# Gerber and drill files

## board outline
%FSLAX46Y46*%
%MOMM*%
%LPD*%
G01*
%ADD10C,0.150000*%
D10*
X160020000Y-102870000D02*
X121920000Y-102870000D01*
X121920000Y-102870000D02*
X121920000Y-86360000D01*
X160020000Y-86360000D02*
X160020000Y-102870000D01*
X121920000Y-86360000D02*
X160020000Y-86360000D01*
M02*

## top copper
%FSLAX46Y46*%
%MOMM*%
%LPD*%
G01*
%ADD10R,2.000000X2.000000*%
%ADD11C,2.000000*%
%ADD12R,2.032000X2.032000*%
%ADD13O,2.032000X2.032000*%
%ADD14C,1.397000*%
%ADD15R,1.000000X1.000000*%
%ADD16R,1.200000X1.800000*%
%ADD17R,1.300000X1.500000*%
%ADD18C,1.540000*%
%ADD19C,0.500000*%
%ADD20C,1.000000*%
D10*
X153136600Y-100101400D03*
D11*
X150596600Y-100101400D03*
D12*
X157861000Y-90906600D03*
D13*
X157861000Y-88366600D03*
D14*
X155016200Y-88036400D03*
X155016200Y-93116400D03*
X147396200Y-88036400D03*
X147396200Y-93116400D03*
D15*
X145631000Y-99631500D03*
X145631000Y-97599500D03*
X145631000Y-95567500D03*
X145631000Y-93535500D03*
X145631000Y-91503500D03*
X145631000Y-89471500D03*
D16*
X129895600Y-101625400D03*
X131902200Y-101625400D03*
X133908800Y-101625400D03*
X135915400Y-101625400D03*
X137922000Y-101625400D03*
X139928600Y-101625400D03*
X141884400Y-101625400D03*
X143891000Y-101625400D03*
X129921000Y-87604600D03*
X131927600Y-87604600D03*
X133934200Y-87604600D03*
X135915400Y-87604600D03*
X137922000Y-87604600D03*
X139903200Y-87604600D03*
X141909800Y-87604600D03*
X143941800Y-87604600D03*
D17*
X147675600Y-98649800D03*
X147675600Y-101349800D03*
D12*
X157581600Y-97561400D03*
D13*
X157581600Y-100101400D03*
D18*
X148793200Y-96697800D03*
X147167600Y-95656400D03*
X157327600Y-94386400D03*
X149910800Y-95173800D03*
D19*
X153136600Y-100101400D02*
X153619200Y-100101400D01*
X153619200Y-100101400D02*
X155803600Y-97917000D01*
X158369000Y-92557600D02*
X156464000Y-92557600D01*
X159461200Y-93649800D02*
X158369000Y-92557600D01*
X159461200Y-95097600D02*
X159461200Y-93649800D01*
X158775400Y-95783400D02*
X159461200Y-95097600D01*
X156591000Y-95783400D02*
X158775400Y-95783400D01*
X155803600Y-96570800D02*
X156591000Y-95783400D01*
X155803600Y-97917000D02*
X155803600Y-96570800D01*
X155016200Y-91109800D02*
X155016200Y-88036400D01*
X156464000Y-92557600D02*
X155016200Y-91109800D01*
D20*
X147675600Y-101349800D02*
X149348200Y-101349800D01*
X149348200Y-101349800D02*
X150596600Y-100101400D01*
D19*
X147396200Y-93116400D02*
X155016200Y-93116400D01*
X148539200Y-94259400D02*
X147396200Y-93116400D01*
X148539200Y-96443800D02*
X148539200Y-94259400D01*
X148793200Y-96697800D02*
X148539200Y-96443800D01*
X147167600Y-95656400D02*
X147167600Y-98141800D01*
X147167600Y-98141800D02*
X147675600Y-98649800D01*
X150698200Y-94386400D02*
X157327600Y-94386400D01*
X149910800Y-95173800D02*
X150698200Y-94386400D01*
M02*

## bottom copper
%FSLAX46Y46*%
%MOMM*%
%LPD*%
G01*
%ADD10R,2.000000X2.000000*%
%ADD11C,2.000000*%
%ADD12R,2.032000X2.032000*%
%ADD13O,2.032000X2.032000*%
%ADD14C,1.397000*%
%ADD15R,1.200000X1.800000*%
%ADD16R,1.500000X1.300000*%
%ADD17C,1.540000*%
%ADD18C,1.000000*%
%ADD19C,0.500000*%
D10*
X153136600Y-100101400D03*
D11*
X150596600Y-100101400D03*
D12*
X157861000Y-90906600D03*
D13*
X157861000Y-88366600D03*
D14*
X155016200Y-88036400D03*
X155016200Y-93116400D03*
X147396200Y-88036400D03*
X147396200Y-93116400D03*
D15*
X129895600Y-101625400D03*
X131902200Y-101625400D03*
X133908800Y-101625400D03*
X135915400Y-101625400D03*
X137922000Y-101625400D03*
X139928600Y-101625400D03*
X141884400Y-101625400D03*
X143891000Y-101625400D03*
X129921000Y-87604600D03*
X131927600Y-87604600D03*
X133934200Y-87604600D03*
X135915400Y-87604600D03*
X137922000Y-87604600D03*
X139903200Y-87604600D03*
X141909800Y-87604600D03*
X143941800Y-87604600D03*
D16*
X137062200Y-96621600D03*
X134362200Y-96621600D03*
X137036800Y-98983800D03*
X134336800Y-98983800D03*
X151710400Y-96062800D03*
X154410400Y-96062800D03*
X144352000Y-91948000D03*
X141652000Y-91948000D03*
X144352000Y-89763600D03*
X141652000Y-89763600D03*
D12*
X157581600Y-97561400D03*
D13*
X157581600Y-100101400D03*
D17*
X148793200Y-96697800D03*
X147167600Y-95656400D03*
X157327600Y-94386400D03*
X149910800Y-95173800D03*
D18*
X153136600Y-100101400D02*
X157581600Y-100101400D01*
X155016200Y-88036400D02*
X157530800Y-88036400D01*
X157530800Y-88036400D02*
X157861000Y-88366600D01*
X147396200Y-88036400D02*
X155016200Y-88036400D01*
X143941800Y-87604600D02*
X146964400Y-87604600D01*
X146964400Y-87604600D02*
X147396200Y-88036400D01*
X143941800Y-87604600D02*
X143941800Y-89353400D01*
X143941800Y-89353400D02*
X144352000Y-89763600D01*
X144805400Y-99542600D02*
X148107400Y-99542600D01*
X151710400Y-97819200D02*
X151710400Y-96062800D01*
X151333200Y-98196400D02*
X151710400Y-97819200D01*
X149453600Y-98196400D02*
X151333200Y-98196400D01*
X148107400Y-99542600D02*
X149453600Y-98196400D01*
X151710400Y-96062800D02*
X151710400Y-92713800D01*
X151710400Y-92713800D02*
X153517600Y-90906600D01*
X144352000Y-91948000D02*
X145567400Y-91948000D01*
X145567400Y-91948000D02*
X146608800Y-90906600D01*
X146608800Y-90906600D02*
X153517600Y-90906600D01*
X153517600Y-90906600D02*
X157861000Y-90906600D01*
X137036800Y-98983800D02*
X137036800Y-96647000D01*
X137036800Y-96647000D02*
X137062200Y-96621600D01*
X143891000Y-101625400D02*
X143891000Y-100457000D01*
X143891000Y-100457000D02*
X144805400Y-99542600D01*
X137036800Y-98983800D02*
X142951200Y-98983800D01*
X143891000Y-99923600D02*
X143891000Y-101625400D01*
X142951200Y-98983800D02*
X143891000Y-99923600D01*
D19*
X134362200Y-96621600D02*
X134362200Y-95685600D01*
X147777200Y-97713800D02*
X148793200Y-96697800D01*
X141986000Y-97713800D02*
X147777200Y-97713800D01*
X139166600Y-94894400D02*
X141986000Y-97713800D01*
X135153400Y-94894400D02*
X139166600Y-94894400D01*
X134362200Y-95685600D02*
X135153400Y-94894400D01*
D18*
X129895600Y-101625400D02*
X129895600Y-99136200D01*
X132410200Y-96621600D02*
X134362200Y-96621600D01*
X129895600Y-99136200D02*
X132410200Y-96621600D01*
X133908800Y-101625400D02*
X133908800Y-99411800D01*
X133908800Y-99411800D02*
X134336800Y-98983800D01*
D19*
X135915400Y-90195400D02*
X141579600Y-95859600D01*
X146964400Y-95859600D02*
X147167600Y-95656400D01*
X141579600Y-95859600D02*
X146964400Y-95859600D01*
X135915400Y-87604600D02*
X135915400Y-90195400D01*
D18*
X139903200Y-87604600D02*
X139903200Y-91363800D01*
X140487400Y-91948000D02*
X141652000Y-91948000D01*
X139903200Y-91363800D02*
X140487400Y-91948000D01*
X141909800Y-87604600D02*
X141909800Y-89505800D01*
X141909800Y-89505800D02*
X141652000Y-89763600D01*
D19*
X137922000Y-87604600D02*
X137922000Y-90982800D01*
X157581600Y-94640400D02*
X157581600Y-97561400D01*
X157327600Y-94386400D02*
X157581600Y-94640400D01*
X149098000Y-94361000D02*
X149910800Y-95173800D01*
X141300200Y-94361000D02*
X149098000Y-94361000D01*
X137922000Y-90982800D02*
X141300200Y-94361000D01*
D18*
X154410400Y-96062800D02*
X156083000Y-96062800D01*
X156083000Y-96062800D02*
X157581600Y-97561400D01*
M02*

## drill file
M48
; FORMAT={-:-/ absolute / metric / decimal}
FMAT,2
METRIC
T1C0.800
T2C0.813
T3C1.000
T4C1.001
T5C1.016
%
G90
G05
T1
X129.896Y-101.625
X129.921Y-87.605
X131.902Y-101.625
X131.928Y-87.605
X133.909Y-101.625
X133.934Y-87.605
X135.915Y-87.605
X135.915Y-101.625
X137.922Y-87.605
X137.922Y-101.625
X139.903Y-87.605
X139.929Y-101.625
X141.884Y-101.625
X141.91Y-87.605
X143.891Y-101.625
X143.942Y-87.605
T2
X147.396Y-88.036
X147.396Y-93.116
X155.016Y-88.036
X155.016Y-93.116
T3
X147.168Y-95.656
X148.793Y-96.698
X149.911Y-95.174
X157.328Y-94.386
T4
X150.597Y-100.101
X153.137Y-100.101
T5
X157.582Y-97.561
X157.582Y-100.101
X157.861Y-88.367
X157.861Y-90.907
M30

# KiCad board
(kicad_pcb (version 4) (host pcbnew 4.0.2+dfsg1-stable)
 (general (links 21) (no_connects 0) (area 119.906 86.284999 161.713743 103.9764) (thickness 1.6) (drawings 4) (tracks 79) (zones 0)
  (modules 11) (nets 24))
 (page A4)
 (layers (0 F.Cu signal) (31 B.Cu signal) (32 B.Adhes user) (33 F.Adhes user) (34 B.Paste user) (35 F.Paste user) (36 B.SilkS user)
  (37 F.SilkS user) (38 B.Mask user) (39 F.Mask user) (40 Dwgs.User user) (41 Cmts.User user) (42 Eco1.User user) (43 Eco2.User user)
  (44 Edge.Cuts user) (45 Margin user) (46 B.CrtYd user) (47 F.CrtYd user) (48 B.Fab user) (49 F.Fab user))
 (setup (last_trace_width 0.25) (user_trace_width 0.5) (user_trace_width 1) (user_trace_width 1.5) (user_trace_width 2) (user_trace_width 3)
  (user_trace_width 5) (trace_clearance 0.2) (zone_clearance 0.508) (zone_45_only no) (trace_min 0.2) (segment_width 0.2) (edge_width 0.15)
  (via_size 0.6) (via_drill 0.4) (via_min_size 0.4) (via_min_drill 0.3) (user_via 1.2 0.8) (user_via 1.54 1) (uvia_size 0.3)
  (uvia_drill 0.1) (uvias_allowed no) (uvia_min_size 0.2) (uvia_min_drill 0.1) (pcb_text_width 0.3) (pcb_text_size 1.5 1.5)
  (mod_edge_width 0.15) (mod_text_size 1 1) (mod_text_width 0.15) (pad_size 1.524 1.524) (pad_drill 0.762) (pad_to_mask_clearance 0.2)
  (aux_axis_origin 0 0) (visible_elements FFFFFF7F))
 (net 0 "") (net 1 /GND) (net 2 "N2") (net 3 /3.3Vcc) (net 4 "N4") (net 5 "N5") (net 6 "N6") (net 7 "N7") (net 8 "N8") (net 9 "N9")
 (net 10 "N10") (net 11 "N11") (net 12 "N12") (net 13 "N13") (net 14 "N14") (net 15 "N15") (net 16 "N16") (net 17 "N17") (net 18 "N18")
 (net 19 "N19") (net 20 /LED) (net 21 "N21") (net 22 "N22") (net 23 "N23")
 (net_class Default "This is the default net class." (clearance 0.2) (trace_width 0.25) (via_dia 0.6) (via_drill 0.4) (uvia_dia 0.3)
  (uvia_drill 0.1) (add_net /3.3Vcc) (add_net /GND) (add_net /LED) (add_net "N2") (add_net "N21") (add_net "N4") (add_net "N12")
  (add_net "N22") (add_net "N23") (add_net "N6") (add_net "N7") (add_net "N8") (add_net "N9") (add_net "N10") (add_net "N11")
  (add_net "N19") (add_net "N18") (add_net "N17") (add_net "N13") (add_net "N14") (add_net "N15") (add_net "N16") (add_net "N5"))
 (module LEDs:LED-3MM (layer F.Cu) (at 153.1366 100.1014 180)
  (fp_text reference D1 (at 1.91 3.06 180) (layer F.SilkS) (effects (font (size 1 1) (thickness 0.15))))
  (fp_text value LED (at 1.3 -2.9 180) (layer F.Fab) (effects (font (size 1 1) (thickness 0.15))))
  (pad 1 thru_hole rect (at 0 0 270) (size 2 2) (drill 1.00076) (layers *.Cu *.Mask F.SilkS) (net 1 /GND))
  (pad 2 thru_hole circle (at 2.54 0 180) (size 2 2) (drill 1.00076) (layers *.Cu *.Mask F.SilkS) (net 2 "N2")))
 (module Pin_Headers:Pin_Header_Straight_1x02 (layer F.Cu) (at 157.861 90.9066 180)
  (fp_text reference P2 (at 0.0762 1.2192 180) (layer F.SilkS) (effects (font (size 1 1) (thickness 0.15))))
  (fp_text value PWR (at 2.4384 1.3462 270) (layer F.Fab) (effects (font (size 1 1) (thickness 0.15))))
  (pad 1 thru_hole rect (at 0 0 180) (size 2.032 2.032) (drill 1.016) (layers *.Cu *.Mask F.SilkS) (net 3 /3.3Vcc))
  (pad 2 thru_hole oval (at 0 2.54 180) (size 2.032 2.032) (drill 1.016) (layers *.Cu *.Mask F.SilkS) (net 1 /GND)))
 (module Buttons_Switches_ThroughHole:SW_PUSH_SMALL (layer F.Cu) (at 151.2062 90.5764)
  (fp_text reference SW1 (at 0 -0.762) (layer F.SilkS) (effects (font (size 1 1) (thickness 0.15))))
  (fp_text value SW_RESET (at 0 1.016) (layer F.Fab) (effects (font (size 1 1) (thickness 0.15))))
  (pad 1 thru_hole circle (at 3.81 -2.54) (size 1.397 1.397) (drill 0.8128) (layers *.Cu *.Mask F.SilkS) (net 1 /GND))
  (pad 2 thru_hole circle (at 3.81 2.54) (size 1.397 1.397) (drill 0.8128) (layers *.Cu *.Mask F.SilkS) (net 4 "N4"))
  (pad 1 thru_hole circle (at -3.81 -2.54) (size 1.397 1.397) (drill 0.8128) (layers *.Cu *.Mask F.SilkS) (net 1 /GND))
  (pad 2 thru_hole circle (at -3.81 2.54) (size 1.397 1.397) (drill 0.8128) (layers *.Cu *.Mask F.SilkS) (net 4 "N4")))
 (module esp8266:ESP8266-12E (layer F.Cu) (at 133.731 94.615 90)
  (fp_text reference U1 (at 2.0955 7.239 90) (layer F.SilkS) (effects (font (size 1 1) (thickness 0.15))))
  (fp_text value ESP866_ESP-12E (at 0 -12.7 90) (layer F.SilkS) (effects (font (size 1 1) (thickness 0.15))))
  (pad 9 smd rect (at -5.0165 11.9 180) (size 1 1) (layers F.Cu F.Paste F.Mask) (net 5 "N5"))
  (pad 10 smd rect (at -2.9845 11.9 180) (size 1 1) (layers F.Cu F.Paste F.Mask) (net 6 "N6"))
  (pad 11 smd rect (at -0.9525 11.9 180) (size 1 1) (layers F.Cu F.Paste F.Mask) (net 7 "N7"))
  (pad 12 smd rect (at 1.0795 11.9 180) (size 1 1) (layers F.Cu F.Paste F.Mask) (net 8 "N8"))
  (pad 13 smd rect (at 3.1115 11.9 180) (size 1 1) (layers F.Cu F.Paste F.Mask) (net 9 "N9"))
  (pad 14 smd rect (at 5.1435 11.9 180) (size 1 1) (layers F.Cu F.Paste F.Mask) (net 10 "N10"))
  (pad 1 thru_hole rect (at -7.0104 -3.8354 90) (size 1.8 1.2) (drill 0.8) (layers *.Cu *.Mask F.SilkS) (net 4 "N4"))
  (pad 2 thru_hole rect (at -7.0104 -1.8288 90) (size 1.8 1.2) (drill 0.8) (layers *.Cu *.Mask F.SilkS) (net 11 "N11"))
  (pad 3 thru_hole rect (at -7.0104 0.1778 90) (size 1.8 1.2) (drill 0.8) (layers *.Cu *.Mask F.SilkS) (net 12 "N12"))
  (pad 4 thru_hole rect (at -7.0104 2.1844 90) (size 1.8 1.2) (drill 0.8) (layers *.Cu *.Mask F.SilkS) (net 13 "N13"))
  (pad 5 thru_hole rect (at -7.0104 4.191 90) (size 1.8 1.2) (drill 0.8) (layers *.Cu *.Mask F.SilkS) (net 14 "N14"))
  (pad 6 thru_hole rect (at -7.0104 6.1976 90) (size 1.8 1.2) (drill 0.8) (layers *.Cu *.Mask F.SilkS) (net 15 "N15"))
  (pad 7 thru_hole rect (at -7.0104 8.1534 90) (size 1.8 1.2) (drill 0.8) (layers *.Cu *.Mask F.SilkS) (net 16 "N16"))
  (pad 8 thru_hole rect (at -7.0104 10.16 90) (size 1.8 1.2) (drill 0.8) (layers *.Cu *.Mask F.SilkS) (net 3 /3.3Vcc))
  (pad 22 thru_hole rect (at 7.0104 -3.81 90) (size 1.8 1.2) (drill 0.8) (layers *.Cu *.Mask F.SilkS) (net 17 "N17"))
  (pad 21 thru_hole rect (at 7.0104 -1.8034 90) (size 1.8 1.2) (drill 0.8) (layers *.Cu *.Mask F.SilkS) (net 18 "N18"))
  (pad 20 thru_hole rect (at 7.0104 0.2032 90) (size 1.8 1.2) (drill 0.8) (layers *.Cu *.Mask F.SilkS) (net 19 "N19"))
  (pad 19 thru_hole rect (at 7.0104 2.1844 90) (size 1.8 1.2) (drill 0.8) (layers *.Cu *.Mask F.SilkS) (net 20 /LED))
  (pad 18 thru_hole rect (at 7.0104 4.191 90) (size 1.8 1.2) (drill 0.8) (layers *.Cu *.Mask F.SilkS) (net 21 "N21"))
  (pad 17 thru_hole rect (at 7.0104 6.1722 90) (size 1.8 1.2) (drill 0.8) (layers *.Cu *.Mask F.SilkS) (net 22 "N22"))
  (pad 16 thru_hole rect (at 7.0104 8.1788 90) (size 1.8 1.2) (drill 0.8) (layers *.Cu *.Mask F.SilkS) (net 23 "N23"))
  (pad 15 thru_hole rect (at 7.0104 10.2108 90) (size 1.8 1.2) (drill 0.8) (layers *.Cu *.Mask F.SilkS) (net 1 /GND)))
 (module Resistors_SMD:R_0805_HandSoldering (layer B.Cu) (at 135.7122 96.6216 180)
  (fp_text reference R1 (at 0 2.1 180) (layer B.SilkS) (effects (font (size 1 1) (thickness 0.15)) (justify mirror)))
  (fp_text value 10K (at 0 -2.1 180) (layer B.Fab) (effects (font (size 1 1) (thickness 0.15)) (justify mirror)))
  (pad 1 smd rect (at -1.35 0 180) (size 1.5 1.3) (layers B.Cu B.Paste B.Mask) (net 3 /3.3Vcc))
  (pad 2 smd rect (at 1.35 0 180) (size 1.5 1.3) (layers B.Cu B.Paste B.Mask) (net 4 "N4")))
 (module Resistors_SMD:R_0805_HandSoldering (layer B.Cu) (at 135.6868 98.9838 180)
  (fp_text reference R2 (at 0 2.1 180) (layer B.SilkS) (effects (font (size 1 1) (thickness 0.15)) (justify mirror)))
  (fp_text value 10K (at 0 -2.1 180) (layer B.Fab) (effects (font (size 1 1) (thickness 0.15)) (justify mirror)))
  (pad 1 smd rect (at -1.35 0 180) (size 1.5 1.3) (layers B.Cu B.Paste B.Mask) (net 3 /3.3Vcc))
  (pad 2 smd rect (at 1.35 0 180) (size 1.5 1.3) (layers B.Cu B.Paste B.Mask) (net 12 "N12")))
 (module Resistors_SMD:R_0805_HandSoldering (layer F.Cu) (at 147.6756 99.9998 270)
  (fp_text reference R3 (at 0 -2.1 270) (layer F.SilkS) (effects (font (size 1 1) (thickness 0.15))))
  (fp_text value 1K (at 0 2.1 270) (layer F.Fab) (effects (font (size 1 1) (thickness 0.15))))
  (pad 1 smd rect (at -1.35 0 270) (size 1.5 1.3) (layers F.Cu F.Paste F.Mask) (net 20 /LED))
  (pad 2 smd rect (at 1.35 0 270) (size 1.5 1.3) (layers F.Cu F.Paste F.Mask) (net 2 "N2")))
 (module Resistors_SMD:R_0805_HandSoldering (layer B.Cu) (at 153.0604 96.0628)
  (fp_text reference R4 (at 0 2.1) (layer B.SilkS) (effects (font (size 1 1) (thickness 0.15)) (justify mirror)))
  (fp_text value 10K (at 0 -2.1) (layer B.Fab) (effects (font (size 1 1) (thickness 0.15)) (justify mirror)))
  (pad 1 smd rect (at -1.35 0) (size 1.5 1.3) (layers B.Cu B.Paste B.Mask) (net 3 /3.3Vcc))
  (pad 2 smd rect (at 1.35 0) (size 1.5 1.3) (layers B.Cu B.Paste B.Mask) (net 21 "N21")))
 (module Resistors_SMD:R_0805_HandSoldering (layer B.Cu) (at 143.002 91.948 180)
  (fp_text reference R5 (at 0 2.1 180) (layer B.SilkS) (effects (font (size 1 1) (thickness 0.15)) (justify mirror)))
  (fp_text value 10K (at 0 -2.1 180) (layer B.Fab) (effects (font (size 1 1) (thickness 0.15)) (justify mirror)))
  (pad 1 smd rect (at -1.35 0 180) (size 1.5 1.3) (layers B.Cu B.Paste B.Mask) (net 3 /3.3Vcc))
  (pad 2 smd rect (at 1.35 0 180) (size 1.5 1.3) (layers B.Cu B.Paste B.Mask) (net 22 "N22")))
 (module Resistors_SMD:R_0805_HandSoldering (layer B.Cu) (at 143.002 89.7636 180)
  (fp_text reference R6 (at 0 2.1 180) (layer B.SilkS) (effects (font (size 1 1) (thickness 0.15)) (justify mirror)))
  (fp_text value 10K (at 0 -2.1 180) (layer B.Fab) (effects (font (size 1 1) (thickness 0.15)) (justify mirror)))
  (pad 1 smd rect (at -1.35 0 180) (size 1.5 1.3) (layers B.Cu B.Paste B.Mask) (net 1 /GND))
  (pad 2 smd rect (at 1.35 0 180) (size 1.5 1.3) (layers B.Cu B.Paste B.Mask) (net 23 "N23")))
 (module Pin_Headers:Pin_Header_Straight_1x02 (layer F.Cu) (at 157.5816 97.5614)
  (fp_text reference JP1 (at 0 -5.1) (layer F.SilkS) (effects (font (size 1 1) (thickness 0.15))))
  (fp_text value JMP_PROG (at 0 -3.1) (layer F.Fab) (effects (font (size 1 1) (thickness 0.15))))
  (pad 1 thru_hole rect (at 0 0) (size 2.032 2.032) (drill 1.016) (layers *.Cu *.Mask F.SilkS) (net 21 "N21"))
  (pad 2 thru_hole oval (at 0 2.54) (size 2.032 2.032) (drill 1.016) (layers *.Cu *.Mask F.SilkS) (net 1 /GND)))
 (gr_line (start 160.02 102.87) (end 121.92 102.87) (angle 90) (layer Edge.Cuts) (width 0.15))
 (gr_line (start 121.92 102.87) (end 121.92 86.36) (angle 90) (layer Edge.Cuts) (width 0.15))
 (gr_line (start 160.02 86.36) (end 160.02 102.87) (angle 90) (layer Edge.Cuts) (width 0.15))
 (gr_line (start 121.92 86.36) (end 160.02 86.36) (angle 90) (layer Edge.Cuts) (width 0.15))
 (segment (start 153.1366 100.1014) (end 153.6192 100.1014) (width 0.5) (layer F.Cu) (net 1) (status 30))
 (segment (start 153.6192 100.1014) (end 155.8036 97.917) (width 0.5) (layer F.Cu) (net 1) (status 10))
 (segment (start 158.369 92.5576) (end 156.464 92.5576) (width 0.5) (layer F.Cu) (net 1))
 (segment (start 159.4612 93.6498) (end 158.369 92.5576) (width 0.5) (layer F.Cu) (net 1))
 (segment (start 159.4612 95.0976) (end 159.4612 93.6498) (width 0.5) (layer F.Cu) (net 1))
 (segment (start 158.7754 95.7834) (end 159.4612 95.0976) (width 0.5) (layer F.Cu) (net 1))
 (segment (start 156.591 95.7834) (end 158.7754 95.7834) (width 0.5) (layer F.Cu) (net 1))
 (segment (start 155.8036 96.5708) (end 156.591 95.7834) (width 0.5) (layer F.Cu) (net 1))
 (segment (start 155.8036 97.917) (end 155.8036 96.5708) (width 0.5) (layer F.Cu) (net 1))
 (segment (start 155.0162 91.1098) (end 155.0162 88.0364) (width 0.5) (layer F.Cu) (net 1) (status 20))
 (segment (start 156.464 92.5576) (end 155.0162 91.1098) (width 0.5) (layer F.Cu) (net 1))
 (segment (start 153.1366 100.1014) (end 157.5816 100.1014) (width 1) (layer B.Cu) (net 1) (status 30))
 (segment (start 155.0162 88.0364) (end 157.5308 88.0364) (width 1) (layer B.Cu) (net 1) (status 30))
 (segment (start 157.5308 88.0364) (end 157.861 88.3666) (width 1) (layer B.Cu) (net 1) (status 30))
 (segment (start 147.3962 88.0364) (end 155.0162 88.0364) (width 1) (layer B.Cu) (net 1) (status 30))
 (segment (start 143.9418 87.6046) (end 146.9644 87.6046) (width 1) (layer B.Cu) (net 1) (status 30))
 (segment (start 146.9644 87.6046) (end 147.3962 88.0364) (width 1) (layer B.Cu) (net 1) (status 30))
 (segment (start 143.9418 87.6046) (end 143.9418 89.3534) (width 1) (layer B.Cu) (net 1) (status 30))
 (segment (start 143.9418 89.3534) (end 144.352 89.7636) (width 1) (layer B.Cu) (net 1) (status 30))
 (segment (start 147.6756 101.3498) (end 149.3482 101.3498) (width 1) (layer F.Cu) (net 2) (status 10))
 (segment (start 149.3482 101.3498) (end 150.5966 100.1014) (width 1) (layer F.Cu) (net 2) (status 20))
 (segment (start 144.8054 99.5426) (end 148.1074 99.5426) (width 1) (layer B.Cu) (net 3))
 (segment (start 151.7104 97.8192) (end 151.7104 96.0628) (width 1) (layer B.Cu) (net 3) (status 20))
 (segment (start 151.3332 98.1964) (end 151.7104 97.8192) (width 1) (layer B.Cu) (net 3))
 (segment (start 149.4536 98.1964) (end 151.3332 98.1964) (width 1) (layer B.Cu) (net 3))
 (segment (start 148.1074 99.5426) (end 149.4536 98.1964) (width 1) (layer B.Cu) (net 3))
 (segment (start 151.7104 96.0628) (end 151.7104 92.7138) (width 1) (layer B.Cu) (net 3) (status 10))
 (segment (start 151.7104 92.7138) (end 153.5176 90.9066) (width 1) (layer B.Cu) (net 3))
 (segment (start 144.352 91.948) (end 145.5674 91.948) (width 1) (layer B.Cu) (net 3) (status 10))
 (segment (start 145.5674 91.948) (end 146.6088 90.9066) (width 1) (layer B.Cu) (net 3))
 (segment (start 146.6088 90.9066) (end 153.5176 90.9066) (width 1) (layer B.Cu) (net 3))
 (segment (start 153.5176 90.9066) (end 157.861 90.9066) (width 1) (layer B.Cu) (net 3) (status 20))
 (segment (start 137.0368 98.9838) (end 137.0368 96.647) (width 1) (layer B.Cu) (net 3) (status 30))
 (segment (start 137.0368 96.647) (end 137.0622 96.6216) (width 1) (layer B.Cu) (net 3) (status 30))
 (segment (start 143.891 101.6254) (end 143.891 100.457) (width 1) (layer B.Cu) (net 3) (status 10))
 (segment (start 143.891 100.457) (end 144.8054 99.5426) (width 1) (layer B.Cu) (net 3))
 (segment (start 137.0368 98.9838) (end 142.9512 98.9838) (width 1) (layer B.Cu) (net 3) (status 10))
 (segment (start 143.891 99.9236) (end 143.891 101.6254) (width 1) (layer B.Cu) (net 3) (status 20))
 (segment (start 142.9512 98.9838) (end 143.891 99.9236) (width 1) (layer B.Cu) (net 3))
 (segment (start 147.3962 93.1164) (end 155.0162 93.1164) (width 0.5) (layer F.Cu) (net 4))
 (segment (start 134.3622 96.6216) (end 134.3622 95.6856) (width 0.5) (layer B.Cu) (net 4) (status 10))
 (segment (start 148.5392 94.2594) (end 147.3962 93.1164) (width 0.5) (layer F.Cu) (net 4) (status 20))
 (segment (start 148.5392 96.4438) (end 148.5392 94.2594) (width 0.5) (layer F.Cu) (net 4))
 (segment (start 148.7932 96.6978) (end 148.5392 96.4438) (width 0.5) (layer F.Cu) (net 4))
 (via (at 148.7932 96.6978) (size 1.54) (drill 1) (layers F.Cu B.Cu) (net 4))
 (segment (start 147.7772 97.7138) (end 148.7932 96.6978) (width 0.5) (layer B.Cu) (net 4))
 (segment (start 141.986 97.7138) (end 147.7772 97.7138) (width 0.5) (layer B.Cu) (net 4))
 (segment (start 139.1666 94.8944) (end 141.986 97.7138) (width 0.5) (layer B.Cu) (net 4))
 (segment (start 135.1534 94.8944) (end 139.1666 94.8944) (width 0.5) (layer B.Cu) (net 4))
 (segment (start 134.3622 95.6856) (end 135.1534 94.8944) (width 0.5) (layer B.Cu) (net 4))
 (segment (start 129.8956 101.6254) (end 129.8956 99.1362) (width 1) (layer B.Cu) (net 4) (status 10))
 (segment (start 132.4102 96.6216) (end 134.3622 96.6216) (width 1) (layer B.Cu) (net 4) (status 20))
 (segment (start 129.8956 99.1362) (end 132.4102 96.6216) (width 1) (layer B.Cu) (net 4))
 (segment (start 133.9088 101.6254) (end 133.9088 99.4118) (width 1) (layer B.Cu) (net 12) (status 30))
 (segment (start 133.9088 99.4118) (end 134.3368 98.9838) (width 1) (layer B.Cu) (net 12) (status 30))
 (segment (start 147.1676 95.6564) (end 147.1676 98.1418) (width 0.5) (layer F.Cu) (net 20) (status 20))
 (segment (start 147.1676 98.1418) (end 147.6756 98.6498) (width 0.5) (layer F.Cu) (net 20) (status 30))
 (segment (start 135.9154 90.1954) (end 141.5796 95.8596) (width 0.5) (layer B.Cu) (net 20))
 (via (at 147.1676 95.6564) (size 1.54) (drill 1) (layers F.Cu B.Cu) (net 20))
 (segment (start 146.9644 95.8596) (end 147.1676 95.6564) (width 0.5) (layer B.Cu) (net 20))
 (segment (start 141.5796 95.8596) (end 146.9644 95.8596) (width 0.5) (layer B.Cu) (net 20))
 (segment (start 135.9154 87.6046) (end 135.9154 90.1954) (width 0.5) (layer B.Cu) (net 20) (status 10))
 (segment (start 139.9032 87.6046) (end 139.9032 91.3638) (width 1) (layer B.Cu) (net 22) (status 10))
 (segment (start 140.4874 91.948) (end 141.652 91.948) (width 1) (layer B.Cu) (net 22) (status 20))
 (segment (start 139.9032 91.3638) (end 140.4874 91.948) (width 1) (layer B.Cu) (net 22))
 (segment (start 141.9098 87.6046) (end 141.9098 89.5058) (width 1) (layer B.Cu) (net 23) (status 30))
 (segment (start 141.9098 89.5058) (end 141.652 89.7636) (width 1) (layer B.Cu) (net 23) (status 30))
 (segment (start 137.922 87.6046) (end 137.922 90.9828) (width 0.5) (layer B.Cu) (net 21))
 (segment (start 157.5816 94.6404) (end 157.5816 97.5614) (width 0.5) (layer B.Cu) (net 21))
 (segment (start 157.3276 94.3864) (end 157.5816 94.6404) (width 0.5) (layer B.Cu) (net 21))
 (via (at 157.3276 94.3864) (size 1.54) (drill 1) (layers F.Cu B.Cu) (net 21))
 (segment (start 150.6982 94.3864) (end 157.3276 94.3864) (width 0.5) (layer F.Cu) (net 21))
 (segment (start 149.9108 95.1738) (end 150.6982 94.3864) (width 0.5) (layer F.Cu) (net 21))
 (via (at 149.9108 95.1738) (size 1.54) (drill 1) (layers F.Cu B.Cu) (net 21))
 (segment (start 149.098 94.361) (end 149.9108 95.1738) (width 0.5) (layer B.Cu) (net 21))
 (segment (start 141.3002 94.361) (end 149.098 94.361) (width 0.5) (layer B.Cu) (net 21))
 (segment (start 137.922 90.9828) (end 141.3002 94.361) (width 0.5) (layer B.Cu) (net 21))
 (segment (start 154.4104 96.0628) (end 156.083 96.0628) (width 1) (layer B.Cu) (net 21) (status 10))
 (segment (start 156.083 96.0628) (end 157.5816 97.5614) (width 1) (layer B.Cu) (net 21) (status 20)))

